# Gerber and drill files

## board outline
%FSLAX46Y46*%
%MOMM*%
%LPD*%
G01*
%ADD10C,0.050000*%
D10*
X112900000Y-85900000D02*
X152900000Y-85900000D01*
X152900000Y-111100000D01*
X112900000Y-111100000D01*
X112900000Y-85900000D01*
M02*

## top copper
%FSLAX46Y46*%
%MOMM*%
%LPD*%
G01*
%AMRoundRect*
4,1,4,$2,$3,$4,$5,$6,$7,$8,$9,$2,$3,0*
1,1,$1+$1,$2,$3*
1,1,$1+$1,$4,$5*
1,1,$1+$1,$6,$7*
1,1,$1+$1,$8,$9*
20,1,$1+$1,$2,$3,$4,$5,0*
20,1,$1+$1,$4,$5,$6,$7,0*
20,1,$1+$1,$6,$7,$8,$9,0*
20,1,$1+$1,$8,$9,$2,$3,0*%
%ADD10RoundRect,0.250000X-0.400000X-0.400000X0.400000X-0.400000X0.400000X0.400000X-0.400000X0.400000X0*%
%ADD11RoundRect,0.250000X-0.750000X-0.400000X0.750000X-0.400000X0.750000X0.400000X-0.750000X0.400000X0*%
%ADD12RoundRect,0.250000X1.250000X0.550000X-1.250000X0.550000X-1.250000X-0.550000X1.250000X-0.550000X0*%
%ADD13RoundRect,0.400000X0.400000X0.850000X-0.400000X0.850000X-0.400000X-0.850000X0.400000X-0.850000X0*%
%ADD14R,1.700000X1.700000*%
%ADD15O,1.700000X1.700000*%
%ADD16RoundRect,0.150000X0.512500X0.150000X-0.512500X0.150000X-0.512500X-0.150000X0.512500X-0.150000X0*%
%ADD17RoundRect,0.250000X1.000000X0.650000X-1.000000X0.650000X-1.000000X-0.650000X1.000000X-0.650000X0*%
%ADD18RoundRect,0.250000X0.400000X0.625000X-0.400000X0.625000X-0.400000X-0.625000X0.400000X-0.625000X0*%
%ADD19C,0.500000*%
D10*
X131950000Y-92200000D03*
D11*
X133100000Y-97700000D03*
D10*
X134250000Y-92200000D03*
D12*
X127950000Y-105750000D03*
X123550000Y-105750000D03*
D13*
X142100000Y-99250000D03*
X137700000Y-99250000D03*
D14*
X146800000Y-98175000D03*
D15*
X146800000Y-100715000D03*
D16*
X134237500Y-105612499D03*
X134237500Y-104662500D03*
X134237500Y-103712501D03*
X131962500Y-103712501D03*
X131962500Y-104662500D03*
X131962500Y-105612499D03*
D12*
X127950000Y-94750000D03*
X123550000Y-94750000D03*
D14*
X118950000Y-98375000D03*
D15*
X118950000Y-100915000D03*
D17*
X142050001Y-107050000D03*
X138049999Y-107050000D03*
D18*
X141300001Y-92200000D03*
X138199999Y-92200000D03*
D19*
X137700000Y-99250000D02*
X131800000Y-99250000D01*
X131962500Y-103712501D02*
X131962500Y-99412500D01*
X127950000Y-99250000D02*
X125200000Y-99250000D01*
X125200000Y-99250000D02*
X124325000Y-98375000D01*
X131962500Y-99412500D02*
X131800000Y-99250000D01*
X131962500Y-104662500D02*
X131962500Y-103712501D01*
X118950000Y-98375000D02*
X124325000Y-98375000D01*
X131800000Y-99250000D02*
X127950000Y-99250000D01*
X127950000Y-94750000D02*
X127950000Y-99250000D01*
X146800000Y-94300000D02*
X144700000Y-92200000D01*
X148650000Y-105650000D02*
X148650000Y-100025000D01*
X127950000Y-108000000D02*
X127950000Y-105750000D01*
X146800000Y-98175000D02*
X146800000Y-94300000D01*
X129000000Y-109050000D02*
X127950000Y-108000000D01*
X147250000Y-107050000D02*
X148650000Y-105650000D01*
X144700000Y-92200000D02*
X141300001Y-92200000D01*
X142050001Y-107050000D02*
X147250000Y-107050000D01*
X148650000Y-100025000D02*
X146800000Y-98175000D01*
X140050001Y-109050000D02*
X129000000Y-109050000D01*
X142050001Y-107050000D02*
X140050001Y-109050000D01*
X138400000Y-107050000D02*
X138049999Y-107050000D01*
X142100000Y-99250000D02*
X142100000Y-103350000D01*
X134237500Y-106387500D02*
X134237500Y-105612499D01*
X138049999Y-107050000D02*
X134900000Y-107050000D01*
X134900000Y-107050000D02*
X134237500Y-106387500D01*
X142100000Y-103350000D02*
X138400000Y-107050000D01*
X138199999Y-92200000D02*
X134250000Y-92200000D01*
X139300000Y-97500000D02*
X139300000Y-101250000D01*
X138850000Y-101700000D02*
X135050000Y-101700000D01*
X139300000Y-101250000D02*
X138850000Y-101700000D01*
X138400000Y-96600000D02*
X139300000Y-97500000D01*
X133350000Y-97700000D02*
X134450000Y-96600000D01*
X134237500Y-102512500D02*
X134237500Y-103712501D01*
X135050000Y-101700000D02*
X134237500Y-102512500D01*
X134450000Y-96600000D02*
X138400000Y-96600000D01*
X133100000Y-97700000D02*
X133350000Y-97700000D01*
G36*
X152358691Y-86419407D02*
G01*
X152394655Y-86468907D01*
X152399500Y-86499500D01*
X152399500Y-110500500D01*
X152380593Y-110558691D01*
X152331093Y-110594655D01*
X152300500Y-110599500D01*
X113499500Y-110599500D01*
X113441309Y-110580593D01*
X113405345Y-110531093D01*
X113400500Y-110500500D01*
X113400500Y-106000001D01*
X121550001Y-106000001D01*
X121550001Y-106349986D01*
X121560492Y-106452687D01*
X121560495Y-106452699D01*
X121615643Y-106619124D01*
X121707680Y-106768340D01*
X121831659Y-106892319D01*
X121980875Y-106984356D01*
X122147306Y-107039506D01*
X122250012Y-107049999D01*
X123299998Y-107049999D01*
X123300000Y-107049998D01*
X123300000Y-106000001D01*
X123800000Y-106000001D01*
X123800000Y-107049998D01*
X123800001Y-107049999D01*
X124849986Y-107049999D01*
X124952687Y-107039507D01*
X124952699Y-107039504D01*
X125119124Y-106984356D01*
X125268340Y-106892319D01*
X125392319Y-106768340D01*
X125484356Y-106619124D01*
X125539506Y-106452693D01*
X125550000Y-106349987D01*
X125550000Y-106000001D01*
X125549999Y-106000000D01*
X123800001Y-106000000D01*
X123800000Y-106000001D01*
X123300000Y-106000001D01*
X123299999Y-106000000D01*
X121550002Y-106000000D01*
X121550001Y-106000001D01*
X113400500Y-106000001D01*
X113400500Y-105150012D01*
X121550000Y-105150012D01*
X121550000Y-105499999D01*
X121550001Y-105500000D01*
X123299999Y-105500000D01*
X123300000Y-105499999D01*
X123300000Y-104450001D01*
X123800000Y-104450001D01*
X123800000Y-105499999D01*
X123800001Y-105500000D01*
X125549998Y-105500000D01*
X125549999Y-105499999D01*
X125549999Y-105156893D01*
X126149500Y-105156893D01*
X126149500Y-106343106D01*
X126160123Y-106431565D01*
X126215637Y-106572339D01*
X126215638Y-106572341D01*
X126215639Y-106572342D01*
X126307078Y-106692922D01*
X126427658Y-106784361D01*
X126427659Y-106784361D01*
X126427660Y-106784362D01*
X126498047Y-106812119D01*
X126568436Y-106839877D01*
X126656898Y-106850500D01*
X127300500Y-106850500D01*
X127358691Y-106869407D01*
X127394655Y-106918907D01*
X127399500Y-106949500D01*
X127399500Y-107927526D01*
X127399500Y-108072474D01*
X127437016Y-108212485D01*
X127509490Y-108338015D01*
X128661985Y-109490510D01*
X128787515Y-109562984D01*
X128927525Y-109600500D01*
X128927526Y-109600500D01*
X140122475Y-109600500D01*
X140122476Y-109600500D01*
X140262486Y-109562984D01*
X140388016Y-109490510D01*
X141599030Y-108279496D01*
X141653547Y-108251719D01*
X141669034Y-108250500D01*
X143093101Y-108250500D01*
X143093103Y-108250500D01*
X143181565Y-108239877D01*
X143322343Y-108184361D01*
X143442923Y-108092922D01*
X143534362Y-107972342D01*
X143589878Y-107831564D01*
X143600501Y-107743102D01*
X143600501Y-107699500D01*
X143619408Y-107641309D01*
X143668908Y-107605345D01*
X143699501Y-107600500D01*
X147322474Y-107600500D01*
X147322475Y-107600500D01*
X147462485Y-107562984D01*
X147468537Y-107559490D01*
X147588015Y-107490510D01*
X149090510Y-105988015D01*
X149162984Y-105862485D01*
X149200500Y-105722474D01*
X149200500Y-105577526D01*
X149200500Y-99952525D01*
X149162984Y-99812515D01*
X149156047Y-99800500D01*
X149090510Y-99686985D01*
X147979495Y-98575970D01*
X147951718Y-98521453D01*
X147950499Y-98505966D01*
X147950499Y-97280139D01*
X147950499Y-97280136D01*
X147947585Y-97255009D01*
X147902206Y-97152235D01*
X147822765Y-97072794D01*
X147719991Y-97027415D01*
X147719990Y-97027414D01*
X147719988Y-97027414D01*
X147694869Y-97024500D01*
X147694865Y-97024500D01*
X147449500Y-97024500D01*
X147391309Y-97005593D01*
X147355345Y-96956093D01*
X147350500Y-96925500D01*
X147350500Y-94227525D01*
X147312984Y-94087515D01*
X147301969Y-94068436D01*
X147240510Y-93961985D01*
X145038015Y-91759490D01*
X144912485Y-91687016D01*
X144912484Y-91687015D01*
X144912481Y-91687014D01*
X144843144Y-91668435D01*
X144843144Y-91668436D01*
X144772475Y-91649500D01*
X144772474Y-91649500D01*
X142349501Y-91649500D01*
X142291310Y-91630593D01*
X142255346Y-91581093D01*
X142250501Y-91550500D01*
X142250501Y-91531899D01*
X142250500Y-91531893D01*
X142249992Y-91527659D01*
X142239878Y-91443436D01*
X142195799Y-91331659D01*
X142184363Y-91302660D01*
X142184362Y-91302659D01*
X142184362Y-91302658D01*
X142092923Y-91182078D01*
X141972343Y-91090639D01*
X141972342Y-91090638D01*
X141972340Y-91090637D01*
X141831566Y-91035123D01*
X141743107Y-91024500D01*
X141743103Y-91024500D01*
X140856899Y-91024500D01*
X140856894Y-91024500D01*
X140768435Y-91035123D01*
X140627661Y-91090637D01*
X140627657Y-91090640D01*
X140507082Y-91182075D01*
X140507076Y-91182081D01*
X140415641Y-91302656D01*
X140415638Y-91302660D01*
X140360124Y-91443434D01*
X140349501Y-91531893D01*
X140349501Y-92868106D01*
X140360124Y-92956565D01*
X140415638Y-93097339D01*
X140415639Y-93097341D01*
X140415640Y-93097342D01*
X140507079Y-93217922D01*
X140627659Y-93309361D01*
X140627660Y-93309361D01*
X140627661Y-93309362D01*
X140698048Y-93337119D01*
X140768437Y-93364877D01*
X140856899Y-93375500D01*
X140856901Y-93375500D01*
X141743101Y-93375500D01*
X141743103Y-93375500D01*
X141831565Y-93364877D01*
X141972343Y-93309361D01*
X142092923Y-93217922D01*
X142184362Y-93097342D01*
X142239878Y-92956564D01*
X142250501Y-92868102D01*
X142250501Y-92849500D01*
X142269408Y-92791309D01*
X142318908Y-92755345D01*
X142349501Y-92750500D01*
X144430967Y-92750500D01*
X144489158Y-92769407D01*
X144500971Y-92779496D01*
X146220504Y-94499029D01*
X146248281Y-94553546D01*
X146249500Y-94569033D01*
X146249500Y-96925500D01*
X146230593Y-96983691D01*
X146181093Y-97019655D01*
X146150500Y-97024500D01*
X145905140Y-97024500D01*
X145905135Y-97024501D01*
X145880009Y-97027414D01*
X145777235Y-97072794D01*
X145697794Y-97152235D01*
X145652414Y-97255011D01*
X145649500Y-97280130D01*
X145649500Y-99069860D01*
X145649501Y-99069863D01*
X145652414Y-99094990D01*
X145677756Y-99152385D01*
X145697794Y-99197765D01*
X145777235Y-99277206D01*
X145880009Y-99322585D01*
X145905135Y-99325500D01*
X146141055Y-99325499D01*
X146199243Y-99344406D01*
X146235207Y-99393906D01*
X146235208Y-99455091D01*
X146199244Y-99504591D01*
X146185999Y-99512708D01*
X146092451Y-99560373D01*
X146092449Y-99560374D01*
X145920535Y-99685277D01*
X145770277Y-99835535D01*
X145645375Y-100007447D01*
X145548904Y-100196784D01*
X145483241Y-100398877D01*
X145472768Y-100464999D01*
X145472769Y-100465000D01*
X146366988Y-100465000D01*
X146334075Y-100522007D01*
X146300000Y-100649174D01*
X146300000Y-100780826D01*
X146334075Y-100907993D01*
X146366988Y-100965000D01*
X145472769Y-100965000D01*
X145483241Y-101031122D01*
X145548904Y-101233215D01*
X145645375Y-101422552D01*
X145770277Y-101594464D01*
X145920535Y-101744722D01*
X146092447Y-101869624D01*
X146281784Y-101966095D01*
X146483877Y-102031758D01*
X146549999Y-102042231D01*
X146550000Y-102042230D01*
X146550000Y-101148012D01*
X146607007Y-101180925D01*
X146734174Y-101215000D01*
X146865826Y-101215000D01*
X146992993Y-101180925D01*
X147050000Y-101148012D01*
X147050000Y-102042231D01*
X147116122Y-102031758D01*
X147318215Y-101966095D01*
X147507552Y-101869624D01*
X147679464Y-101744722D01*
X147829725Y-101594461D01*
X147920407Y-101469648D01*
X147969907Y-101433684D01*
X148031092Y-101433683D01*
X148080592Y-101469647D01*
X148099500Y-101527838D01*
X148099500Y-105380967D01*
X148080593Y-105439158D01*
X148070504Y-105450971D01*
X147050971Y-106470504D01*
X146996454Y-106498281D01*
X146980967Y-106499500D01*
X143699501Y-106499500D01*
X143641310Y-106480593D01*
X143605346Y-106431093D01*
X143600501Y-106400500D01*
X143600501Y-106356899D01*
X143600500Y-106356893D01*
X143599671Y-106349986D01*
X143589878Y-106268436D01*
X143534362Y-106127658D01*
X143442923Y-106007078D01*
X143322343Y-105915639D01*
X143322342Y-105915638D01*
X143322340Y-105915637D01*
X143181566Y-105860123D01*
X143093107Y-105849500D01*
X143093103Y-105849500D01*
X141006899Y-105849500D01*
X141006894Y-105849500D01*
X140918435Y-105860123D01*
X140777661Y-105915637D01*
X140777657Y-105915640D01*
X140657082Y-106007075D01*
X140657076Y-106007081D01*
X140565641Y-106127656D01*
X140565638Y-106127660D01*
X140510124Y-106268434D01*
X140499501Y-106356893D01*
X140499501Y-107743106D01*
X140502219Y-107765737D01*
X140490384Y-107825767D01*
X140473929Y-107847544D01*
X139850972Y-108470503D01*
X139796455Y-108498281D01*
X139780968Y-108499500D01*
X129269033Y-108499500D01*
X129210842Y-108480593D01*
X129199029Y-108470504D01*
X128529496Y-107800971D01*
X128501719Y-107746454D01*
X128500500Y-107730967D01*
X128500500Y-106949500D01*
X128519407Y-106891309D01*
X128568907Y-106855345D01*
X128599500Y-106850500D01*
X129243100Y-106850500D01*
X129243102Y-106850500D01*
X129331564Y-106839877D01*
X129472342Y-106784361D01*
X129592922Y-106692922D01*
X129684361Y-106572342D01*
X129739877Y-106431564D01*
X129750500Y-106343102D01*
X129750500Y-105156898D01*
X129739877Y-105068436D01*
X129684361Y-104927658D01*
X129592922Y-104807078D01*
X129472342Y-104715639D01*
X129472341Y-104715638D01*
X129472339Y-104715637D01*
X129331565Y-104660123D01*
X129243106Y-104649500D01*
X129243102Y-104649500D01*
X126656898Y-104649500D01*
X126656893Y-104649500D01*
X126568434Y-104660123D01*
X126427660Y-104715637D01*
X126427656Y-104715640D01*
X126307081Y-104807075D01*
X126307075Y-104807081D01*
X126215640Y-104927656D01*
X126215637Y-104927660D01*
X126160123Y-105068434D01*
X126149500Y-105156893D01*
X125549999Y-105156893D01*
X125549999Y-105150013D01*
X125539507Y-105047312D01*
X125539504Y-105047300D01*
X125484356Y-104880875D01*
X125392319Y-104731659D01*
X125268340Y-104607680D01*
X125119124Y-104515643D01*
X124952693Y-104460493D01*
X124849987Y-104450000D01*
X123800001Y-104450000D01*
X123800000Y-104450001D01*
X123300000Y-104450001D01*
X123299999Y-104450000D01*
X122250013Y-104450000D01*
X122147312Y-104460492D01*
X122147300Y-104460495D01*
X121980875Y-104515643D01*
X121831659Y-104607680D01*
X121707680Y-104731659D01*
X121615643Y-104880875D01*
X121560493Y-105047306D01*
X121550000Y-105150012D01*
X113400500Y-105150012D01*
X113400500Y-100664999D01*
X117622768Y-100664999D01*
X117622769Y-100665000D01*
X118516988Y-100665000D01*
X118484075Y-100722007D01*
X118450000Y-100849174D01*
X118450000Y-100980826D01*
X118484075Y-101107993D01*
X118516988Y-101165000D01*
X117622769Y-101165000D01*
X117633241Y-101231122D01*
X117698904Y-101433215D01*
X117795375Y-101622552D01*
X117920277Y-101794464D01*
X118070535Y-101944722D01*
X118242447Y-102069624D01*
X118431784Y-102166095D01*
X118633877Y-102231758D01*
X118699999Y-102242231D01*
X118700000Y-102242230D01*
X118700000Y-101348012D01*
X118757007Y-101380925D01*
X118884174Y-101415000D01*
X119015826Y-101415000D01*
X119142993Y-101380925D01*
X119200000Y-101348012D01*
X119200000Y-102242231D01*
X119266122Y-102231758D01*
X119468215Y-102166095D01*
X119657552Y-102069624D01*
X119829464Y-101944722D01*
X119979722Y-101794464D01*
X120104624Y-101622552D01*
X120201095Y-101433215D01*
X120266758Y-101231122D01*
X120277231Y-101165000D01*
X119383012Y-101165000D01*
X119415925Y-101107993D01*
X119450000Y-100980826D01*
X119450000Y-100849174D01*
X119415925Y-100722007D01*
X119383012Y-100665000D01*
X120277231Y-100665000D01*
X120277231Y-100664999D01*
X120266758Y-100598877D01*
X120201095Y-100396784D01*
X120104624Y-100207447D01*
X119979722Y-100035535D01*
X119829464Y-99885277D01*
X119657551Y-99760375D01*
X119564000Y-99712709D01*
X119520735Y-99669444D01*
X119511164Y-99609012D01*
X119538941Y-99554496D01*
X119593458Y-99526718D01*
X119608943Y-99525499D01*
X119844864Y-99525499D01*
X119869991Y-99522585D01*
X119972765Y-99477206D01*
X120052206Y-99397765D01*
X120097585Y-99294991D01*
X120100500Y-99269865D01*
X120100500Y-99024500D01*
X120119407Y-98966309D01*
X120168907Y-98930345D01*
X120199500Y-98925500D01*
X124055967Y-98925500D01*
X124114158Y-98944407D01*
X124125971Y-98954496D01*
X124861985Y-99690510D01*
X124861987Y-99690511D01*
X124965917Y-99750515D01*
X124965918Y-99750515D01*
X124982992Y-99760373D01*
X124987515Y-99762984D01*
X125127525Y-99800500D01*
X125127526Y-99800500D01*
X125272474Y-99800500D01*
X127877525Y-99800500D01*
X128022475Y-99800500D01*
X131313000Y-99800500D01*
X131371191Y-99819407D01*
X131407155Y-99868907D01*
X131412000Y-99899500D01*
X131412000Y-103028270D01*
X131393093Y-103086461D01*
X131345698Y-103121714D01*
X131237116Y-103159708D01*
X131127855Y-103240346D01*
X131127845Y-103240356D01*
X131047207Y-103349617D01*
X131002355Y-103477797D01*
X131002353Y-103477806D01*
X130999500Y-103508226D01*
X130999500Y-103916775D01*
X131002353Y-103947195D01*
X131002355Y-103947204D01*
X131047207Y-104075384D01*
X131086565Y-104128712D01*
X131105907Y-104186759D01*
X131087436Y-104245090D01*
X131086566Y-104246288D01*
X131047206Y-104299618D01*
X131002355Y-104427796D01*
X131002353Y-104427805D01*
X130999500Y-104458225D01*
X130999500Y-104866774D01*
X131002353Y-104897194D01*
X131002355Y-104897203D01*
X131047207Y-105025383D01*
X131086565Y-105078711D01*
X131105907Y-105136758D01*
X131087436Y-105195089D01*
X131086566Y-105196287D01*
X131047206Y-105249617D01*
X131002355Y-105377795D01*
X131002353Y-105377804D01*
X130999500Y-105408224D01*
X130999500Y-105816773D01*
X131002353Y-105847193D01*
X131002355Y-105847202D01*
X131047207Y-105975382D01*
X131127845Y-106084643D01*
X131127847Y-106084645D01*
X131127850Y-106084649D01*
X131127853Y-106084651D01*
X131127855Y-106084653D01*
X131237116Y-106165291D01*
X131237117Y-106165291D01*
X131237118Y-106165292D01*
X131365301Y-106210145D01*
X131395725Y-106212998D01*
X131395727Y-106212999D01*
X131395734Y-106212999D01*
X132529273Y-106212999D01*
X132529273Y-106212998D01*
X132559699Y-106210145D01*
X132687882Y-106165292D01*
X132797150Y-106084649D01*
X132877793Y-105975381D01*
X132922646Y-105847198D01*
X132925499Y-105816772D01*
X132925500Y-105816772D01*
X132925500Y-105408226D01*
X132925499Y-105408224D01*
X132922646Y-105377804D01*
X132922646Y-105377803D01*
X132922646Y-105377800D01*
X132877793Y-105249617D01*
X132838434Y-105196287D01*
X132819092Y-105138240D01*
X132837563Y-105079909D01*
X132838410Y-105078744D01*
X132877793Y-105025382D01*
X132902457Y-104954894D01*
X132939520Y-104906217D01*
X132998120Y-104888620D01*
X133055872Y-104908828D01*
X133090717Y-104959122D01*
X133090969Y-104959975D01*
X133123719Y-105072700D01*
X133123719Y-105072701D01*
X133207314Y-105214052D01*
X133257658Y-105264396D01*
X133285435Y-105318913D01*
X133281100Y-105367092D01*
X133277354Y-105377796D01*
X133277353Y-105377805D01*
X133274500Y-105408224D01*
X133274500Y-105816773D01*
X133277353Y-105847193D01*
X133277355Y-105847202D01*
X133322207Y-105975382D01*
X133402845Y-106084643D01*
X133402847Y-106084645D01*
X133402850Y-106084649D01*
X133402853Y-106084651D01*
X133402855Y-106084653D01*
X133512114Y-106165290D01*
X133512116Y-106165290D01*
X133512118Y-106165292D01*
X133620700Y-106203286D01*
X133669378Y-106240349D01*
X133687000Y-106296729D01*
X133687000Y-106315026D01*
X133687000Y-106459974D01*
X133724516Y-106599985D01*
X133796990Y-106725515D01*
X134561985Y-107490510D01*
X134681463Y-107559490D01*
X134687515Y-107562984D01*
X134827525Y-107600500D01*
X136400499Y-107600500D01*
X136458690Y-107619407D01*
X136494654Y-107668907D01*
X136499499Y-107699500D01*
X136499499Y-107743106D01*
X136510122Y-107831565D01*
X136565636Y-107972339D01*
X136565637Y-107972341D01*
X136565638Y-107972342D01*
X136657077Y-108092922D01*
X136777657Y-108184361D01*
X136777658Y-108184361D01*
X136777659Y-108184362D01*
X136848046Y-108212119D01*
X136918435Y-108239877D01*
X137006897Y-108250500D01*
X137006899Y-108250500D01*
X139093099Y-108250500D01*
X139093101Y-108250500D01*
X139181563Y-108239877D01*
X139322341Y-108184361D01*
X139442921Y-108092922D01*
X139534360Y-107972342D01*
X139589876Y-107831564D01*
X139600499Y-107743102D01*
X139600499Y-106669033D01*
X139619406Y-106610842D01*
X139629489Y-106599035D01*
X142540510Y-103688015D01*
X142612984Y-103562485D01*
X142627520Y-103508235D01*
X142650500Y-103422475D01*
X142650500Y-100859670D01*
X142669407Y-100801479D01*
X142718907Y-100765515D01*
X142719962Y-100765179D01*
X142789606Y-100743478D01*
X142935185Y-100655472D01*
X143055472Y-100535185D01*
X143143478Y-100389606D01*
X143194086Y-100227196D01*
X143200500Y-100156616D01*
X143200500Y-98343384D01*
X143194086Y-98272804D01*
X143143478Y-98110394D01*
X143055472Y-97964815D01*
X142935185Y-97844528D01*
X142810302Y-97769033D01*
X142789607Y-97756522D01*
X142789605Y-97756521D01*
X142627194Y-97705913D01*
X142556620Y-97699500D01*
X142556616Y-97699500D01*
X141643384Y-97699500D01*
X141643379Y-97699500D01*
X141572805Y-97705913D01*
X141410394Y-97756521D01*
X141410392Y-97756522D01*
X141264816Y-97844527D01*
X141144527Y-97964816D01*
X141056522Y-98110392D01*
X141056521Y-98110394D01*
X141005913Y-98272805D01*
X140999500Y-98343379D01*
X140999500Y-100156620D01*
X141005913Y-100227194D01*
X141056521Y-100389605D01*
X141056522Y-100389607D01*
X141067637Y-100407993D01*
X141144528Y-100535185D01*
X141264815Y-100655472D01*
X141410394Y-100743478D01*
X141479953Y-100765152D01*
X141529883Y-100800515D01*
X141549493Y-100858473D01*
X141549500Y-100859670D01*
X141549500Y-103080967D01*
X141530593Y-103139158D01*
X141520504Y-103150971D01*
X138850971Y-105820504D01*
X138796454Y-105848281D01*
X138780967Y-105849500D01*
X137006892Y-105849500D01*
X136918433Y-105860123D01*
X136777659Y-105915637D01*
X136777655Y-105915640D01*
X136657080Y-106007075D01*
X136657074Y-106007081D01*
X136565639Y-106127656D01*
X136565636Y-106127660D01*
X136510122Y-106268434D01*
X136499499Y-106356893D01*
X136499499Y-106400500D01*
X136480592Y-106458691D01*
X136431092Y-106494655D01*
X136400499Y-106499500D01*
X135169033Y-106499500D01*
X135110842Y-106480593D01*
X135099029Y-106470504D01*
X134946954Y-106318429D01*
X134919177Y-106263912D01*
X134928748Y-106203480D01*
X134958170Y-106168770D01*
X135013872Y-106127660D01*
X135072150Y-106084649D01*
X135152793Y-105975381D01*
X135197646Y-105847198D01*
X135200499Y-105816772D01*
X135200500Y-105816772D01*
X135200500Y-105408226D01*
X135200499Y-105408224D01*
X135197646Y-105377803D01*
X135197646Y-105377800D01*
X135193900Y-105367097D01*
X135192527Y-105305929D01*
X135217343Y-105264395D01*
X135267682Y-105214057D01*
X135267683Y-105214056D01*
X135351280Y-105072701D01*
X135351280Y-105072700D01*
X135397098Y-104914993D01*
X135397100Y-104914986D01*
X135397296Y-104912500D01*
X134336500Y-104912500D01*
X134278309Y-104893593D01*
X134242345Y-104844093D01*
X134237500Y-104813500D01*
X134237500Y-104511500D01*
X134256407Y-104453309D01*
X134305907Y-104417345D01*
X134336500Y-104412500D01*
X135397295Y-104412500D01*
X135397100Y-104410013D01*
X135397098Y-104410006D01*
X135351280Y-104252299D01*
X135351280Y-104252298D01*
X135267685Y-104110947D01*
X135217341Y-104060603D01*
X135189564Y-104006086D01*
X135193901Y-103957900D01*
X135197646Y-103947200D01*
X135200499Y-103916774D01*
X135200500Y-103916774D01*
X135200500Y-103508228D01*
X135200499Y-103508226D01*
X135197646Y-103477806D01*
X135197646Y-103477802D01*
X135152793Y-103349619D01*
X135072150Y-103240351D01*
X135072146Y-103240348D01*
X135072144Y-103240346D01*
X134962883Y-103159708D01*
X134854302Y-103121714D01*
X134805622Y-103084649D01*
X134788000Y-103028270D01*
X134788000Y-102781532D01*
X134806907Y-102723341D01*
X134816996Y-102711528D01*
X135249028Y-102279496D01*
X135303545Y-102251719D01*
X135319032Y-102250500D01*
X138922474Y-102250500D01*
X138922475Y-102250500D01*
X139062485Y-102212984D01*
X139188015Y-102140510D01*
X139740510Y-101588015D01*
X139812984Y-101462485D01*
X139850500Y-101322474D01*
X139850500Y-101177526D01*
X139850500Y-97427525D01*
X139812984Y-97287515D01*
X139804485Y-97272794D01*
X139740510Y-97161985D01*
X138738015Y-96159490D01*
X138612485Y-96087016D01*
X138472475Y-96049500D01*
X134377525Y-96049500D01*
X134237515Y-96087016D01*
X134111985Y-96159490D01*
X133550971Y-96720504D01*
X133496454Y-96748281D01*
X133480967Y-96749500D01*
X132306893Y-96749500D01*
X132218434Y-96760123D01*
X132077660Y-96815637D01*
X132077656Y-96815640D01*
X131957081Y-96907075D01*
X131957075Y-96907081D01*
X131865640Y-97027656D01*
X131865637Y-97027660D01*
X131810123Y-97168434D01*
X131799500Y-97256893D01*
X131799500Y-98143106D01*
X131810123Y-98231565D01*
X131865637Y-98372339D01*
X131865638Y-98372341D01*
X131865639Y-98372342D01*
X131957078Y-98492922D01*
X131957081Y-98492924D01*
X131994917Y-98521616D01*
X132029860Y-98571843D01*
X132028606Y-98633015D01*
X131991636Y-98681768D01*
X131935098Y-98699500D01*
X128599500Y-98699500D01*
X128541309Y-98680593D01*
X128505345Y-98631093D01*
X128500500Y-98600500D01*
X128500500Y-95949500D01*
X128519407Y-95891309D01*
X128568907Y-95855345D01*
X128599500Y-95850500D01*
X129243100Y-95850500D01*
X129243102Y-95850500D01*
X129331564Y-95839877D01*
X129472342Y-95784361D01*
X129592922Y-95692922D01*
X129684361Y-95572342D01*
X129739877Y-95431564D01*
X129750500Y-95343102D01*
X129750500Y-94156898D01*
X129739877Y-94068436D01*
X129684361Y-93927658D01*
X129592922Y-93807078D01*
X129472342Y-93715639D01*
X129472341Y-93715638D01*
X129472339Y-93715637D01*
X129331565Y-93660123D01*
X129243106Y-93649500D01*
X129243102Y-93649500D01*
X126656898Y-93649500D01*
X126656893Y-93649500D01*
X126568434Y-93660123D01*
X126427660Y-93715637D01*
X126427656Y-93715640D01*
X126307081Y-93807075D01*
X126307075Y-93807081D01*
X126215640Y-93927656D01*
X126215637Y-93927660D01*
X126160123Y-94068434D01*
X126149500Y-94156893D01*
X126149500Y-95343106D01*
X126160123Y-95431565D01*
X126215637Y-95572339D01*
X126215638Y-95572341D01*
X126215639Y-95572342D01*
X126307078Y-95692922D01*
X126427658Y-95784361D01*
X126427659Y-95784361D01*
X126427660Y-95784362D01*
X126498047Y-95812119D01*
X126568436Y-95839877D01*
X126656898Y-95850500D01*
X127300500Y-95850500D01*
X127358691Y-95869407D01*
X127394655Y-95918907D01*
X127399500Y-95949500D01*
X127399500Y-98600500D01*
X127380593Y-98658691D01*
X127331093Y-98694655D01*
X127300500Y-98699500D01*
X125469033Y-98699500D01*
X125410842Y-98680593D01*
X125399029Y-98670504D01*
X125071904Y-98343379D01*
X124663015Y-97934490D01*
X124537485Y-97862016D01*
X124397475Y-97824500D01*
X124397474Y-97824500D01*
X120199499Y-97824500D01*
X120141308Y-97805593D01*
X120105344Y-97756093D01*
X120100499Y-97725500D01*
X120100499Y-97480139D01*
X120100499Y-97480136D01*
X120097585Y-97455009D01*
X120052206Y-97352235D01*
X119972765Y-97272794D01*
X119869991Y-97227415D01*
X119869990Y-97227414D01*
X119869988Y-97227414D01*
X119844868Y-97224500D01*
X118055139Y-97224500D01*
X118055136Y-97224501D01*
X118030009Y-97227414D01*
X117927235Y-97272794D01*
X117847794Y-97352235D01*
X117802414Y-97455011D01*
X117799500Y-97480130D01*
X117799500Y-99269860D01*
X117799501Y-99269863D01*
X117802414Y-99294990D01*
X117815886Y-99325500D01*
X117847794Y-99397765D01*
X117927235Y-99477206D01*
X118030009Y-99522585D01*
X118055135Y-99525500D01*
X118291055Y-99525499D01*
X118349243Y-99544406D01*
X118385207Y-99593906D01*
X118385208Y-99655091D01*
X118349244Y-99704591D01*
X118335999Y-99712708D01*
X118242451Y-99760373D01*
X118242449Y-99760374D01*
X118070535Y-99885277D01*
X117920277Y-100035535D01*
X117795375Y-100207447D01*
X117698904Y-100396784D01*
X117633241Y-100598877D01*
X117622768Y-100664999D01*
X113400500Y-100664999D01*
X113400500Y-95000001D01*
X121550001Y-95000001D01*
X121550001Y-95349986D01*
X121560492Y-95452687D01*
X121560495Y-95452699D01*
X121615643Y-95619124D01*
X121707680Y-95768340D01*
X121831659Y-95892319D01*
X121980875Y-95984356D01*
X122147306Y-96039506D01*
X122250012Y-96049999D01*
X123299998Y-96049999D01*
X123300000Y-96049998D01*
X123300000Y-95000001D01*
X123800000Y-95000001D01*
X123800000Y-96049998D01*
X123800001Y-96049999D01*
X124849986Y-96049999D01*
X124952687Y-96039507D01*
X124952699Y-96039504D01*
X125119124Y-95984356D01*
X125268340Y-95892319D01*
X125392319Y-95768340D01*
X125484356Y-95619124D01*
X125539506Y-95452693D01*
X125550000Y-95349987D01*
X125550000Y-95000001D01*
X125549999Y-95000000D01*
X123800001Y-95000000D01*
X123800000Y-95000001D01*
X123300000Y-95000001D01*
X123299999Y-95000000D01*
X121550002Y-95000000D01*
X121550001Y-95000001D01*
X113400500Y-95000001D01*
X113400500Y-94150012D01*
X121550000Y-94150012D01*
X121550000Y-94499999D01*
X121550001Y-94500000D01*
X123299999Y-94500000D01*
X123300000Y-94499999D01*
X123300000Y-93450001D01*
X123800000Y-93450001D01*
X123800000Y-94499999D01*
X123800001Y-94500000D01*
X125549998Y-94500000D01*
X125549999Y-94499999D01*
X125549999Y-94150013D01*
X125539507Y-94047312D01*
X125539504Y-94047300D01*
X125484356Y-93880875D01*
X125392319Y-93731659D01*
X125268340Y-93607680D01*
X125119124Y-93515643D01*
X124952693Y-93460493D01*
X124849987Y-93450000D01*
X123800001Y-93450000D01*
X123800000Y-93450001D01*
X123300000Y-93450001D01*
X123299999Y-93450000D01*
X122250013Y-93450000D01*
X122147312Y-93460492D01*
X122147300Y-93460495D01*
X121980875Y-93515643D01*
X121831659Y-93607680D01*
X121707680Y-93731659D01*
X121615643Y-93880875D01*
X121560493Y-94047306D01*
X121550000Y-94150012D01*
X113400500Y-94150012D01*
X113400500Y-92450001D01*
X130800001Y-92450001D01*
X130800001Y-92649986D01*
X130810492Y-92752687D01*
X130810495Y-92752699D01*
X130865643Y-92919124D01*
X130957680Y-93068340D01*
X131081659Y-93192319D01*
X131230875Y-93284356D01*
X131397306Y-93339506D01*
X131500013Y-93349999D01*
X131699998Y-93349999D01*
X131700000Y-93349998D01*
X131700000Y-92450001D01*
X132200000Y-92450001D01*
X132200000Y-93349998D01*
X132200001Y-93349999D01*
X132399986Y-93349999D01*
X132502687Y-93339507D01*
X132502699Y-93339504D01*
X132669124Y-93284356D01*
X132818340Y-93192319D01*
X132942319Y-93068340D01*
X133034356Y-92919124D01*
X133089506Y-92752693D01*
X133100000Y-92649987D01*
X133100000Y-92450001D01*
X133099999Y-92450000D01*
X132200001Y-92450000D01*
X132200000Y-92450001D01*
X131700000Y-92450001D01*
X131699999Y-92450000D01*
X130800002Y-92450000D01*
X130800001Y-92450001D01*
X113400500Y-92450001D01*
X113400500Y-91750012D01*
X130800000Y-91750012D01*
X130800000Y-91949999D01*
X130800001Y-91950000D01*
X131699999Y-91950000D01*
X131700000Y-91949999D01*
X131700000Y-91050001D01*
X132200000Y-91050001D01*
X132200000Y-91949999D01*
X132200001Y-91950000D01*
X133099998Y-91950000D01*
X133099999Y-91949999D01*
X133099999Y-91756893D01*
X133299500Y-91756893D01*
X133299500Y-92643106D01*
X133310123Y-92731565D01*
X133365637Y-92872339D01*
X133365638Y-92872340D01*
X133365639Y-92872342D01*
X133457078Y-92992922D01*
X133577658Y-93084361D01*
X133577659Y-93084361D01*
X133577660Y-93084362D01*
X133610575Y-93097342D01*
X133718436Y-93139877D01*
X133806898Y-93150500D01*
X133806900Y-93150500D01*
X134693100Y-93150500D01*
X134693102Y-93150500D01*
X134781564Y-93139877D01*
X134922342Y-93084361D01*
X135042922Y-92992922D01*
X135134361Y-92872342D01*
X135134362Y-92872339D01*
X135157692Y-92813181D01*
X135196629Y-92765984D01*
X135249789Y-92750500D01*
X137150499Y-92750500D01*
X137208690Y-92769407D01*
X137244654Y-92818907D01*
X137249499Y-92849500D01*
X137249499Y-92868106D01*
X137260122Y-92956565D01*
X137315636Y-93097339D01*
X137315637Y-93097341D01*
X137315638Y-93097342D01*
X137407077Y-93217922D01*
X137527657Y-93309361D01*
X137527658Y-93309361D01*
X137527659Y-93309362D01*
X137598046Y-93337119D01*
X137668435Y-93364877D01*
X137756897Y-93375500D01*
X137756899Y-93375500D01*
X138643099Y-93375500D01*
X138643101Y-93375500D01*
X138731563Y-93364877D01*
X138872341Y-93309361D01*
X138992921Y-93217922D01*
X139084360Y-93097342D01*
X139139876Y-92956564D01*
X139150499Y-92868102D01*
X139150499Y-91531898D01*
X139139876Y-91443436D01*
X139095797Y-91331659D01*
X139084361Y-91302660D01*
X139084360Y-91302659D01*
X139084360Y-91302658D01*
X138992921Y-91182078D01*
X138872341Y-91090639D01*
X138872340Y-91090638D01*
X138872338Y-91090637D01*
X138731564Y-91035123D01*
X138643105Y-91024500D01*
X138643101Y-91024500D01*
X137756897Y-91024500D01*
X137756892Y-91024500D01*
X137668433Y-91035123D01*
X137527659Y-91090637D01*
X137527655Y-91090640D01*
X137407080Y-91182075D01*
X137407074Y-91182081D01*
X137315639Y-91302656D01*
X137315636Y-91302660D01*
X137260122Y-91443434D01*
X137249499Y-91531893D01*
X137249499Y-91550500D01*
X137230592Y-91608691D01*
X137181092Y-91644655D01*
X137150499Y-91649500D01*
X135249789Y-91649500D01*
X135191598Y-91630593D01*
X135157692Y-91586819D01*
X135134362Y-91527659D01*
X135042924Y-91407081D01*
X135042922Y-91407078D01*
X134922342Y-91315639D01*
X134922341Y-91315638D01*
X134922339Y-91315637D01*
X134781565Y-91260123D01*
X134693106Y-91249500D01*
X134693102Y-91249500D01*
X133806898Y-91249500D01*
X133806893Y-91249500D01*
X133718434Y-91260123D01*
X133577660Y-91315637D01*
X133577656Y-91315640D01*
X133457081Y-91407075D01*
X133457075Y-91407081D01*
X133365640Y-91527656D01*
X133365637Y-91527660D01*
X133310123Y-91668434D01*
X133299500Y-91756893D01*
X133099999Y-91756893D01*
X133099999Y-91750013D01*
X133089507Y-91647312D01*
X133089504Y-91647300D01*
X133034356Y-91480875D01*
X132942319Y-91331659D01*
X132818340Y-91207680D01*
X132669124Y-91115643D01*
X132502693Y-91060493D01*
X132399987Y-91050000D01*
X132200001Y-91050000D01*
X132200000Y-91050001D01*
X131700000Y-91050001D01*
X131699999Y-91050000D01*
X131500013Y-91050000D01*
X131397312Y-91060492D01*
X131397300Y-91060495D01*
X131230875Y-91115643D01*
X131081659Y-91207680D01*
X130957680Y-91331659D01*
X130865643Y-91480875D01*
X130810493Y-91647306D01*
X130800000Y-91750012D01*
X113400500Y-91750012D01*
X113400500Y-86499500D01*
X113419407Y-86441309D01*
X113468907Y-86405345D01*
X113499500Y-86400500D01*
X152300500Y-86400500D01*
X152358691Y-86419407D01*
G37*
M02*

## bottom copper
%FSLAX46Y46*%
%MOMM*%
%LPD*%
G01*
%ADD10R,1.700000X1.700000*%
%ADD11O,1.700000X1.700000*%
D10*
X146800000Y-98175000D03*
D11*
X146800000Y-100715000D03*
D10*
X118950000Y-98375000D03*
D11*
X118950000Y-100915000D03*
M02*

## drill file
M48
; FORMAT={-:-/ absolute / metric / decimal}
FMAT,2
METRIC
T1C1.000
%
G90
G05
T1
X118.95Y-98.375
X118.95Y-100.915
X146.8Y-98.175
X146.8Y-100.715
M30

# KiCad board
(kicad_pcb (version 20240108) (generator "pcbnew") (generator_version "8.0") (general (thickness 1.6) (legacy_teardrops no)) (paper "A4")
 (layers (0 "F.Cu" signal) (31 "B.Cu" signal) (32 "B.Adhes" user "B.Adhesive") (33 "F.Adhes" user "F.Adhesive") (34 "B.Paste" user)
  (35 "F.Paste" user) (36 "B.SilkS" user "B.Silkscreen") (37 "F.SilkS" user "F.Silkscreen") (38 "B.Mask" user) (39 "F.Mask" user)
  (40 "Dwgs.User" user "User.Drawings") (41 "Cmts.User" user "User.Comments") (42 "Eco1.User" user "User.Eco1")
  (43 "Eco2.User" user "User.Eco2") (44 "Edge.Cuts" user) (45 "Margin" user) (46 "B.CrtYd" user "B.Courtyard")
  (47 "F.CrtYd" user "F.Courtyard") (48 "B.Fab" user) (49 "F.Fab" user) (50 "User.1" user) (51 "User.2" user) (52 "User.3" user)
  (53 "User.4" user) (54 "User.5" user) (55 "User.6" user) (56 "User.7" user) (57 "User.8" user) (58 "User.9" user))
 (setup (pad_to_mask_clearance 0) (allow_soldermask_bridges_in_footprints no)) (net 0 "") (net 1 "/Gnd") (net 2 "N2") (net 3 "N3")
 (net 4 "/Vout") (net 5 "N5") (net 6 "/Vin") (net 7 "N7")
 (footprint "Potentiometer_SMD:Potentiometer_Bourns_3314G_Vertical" (layer "F.Cu") (at 133.1 94.95)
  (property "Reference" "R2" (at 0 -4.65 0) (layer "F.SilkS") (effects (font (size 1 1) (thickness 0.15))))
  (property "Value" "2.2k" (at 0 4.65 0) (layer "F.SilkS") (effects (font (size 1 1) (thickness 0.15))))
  (pad "1" smd roundrect (at -1.15 -2.75) (size 1.3 1.3) (layers "F.Cu" "F.Paste" "F.Mask") (roundrect_rratio 0.1923076923) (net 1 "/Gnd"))
  (pad "2" smd roundrect (at 0 2.75) (size 2 1.3) (layers "F.Cu" "F.Paste" "F.Mask") (roundrect_rratio 0.1923076923) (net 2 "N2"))
  (pad "3" smd roundrect (at 1.15 -2.75) (size 1.3 1.3) (layers "F.Cu" "F.Paste" "F.Mask") (roundrect_rratio 0.1923076923) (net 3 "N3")))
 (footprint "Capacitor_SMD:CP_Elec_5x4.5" (layer "F.Cu") (at 125.75 105.75 180)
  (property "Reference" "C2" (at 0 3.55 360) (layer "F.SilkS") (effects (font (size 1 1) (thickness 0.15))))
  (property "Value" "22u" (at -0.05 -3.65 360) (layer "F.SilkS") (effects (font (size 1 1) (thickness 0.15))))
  (pad "1" smd roundrect (at -2.2 0 180) (size 3 1.6) (layers "F.Cu" "F.Paste" "F.Mask") (roundrect_rratio 0.15625) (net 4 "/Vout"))
  (pad "2" smd roundrect (at 2.2 0 180) (size 3 1.6) (layers "F.Cu" "F.Paste" "F.Mask") (roundrect_rratio 0.15625) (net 1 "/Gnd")))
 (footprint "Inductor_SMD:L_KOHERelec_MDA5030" (layer "F.Cu") (at 139.9 99.25 180)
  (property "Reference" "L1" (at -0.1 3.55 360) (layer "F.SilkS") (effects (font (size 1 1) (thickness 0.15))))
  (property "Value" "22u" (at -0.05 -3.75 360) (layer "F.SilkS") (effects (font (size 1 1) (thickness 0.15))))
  (pad "1" smd roundrect (at -2.2 0 180) (size 1.6 2.5) (layers "F.Cu" "F.Paste" "F.Mask") (roundrect_rratio 0.25) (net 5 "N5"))
  (pad "2" smd roundrect (at 2.2 0 180) (size 1.6 2.5) (layers "F.Cu" "F.Paste" "F.Mask") (roundrect_rratio 0.25) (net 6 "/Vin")))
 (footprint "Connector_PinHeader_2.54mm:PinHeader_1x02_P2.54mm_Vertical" (layer "F.Cu") (at 146.8 98.175)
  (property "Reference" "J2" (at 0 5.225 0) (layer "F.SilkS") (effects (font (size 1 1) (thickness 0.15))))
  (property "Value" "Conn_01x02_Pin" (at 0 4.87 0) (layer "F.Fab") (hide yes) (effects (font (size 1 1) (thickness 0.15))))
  (pad "1" thru_hole rect (at 0 0) (size 1.7 1.7) (drill 1) (layers "*.Cu" "*.Mask") (remove_unused_layers no) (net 4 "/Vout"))
  (pad "2" thru_hole oval (at 0 2.54) (size 1.7 1.7) (drill 1) (layers "*.Cu" "*.Mask") (remove_unused_layers no) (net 1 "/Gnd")))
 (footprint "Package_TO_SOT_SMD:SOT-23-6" (layer "F.Cu") (at 133.1 104.6625 180)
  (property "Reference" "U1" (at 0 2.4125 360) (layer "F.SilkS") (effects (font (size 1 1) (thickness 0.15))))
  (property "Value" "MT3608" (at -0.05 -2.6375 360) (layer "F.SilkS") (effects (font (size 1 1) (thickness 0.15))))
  (pad "1" smd roundrect (at -1.1375 -0.949999 180) (size 1.325 0.6) (layers "F.Cu" "F.Paste" "F.Mask") (roundrect_rratio 0.25) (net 5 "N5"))
  (pad "2" smd roundrect (at -1.1375 0 180) (size 1.325 0.6) (layers "F.Cu" "F.Paste" "F.Mask") (roundrect_rratio 0.25) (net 1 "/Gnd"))
  (pad "3" smd roundrect (at -1.1375 0.949999 180) (size 1.325 0.6) (layers "F.Cu" "F.Paste" "F.Mask") (roundrect_rratio 0.25) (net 2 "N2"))
  (pad "4" smd roundrect (at 1.1375 0.949999 180) (size 1.325 0.6) (layers "F.Cu" "F.Paste" "F.Mask") (roundrect_rratio 0.25) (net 6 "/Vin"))
  (pad "5" smd roundrect (at 1.1375 0 180) (size 1.325 0.6) (layers "F.Cu" "F.Paste" "F.Mask") (roundrect_rratio 0.25) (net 6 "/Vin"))
  (pad "6" smd roundrect (at 1.1375 -0.949999 180) (size 1.325 0.6) (layers "F.Cu" "F.Paste" "F.Mask") (roundrect_rratio 0.25) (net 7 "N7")))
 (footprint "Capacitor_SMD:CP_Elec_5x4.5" (layer "F.Cu") (at 125.75 94.75 180)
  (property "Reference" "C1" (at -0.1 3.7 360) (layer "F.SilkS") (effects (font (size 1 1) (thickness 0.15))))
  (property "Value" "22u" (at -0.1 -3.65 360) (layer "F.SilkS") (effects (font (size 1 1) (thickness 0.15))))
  (pad "1" smd roundrect (at -2.2 0 180) (size 3 1.6) (layers "F.Cu" "F.Paste" "F.Mask") (roundrect_rratio 0.15625) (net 6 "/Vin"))
  (pad "2" smd roundrect (at 2.2 0 180) (size 3 1.6) (layers "F.Cu" "F.Paste" "F.Mask") (roundrect_rratio 0.15625) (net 1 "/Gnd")))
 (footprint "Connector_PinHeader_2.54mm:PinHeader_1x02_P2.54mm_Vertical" (layer "F.Cu") (at 118.95 98.375)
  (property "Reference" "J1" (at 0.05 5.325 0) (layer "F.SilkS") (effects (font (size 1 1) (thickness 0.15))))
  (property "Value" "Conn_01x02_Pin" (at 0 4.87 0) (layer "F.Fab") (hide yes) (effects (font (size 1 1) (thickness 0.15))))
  (pad "1" thru_hole rect (at 0 0) (size 1.7 1.7) (drill 1) (layers "*.Cu" "*.Mask") (remove_unused_layers no) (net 6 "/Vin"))
  (pad "2" thru_hole oval (at 0 2.54) (size 1.7 1.7) (drill 1) (layers "*.Cu" "*.Mask") (remove_unused_layers no) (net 1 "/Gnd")))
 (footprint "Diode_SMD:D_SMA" (layer "F.Cu") (at 140.05 107.05 180)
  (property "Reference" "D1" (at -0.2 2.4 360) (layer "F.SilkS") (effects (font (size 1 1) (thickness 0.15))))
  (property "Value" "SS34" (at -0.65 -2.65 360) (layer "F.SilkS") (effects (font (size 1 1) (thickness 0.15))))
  (pad "1" smd roundrect (at -2.000001 0 180) (size 2.5 1.8) (layers "F.Cu" "F.Paste" "F.Mask") (roundrect_rratio 0.1388888889)
   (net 4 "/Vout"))
  (pad "2" smd roundrect (at 2.000001 0 180) (size 2.5 1.8) (layers "F.Cu" "F.Paste" "F.Mask") (roundrect_rratio 0.1388888889) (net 5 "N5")))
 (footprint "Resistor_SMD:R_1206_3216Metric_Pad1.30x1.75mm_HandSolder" (layer "F.Cu") (at 139.75 92.2 180)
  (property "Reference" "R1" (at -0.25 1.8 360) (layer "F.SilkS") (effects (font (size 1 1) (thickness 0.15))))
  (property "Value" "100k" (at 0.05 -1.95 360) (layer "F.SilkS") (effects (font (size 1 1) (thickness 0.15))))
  (pad "1" smd roundrect (at -1.550001 0 180) (size 1.3 1.75) (layers "F.Cu" "F.Paste" "F.Mask") (roundrect_rratio 0.192308) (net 4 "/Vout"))
  (pad "2" smd roundrect (at 1.550001 0 180) (size 1.3 1.75) (layers "F.Cu" "F.Paste" "F.Mask") (roundrect_rratio 0.192308) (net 3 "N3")))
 (gr_rect (start 112.9 85.9) (end 152.9 111.1) (stroke (width 0.05) (type default)) (fill none) (layer "Edge.Cuts"))
 (segment (start 137.7 99.25) (end 131.8 99.25) (width 0.5) (layer "F.Cu") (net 6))
 (segment (start 131.9625 103.712501) (end 131.9625 99.4125) (width 0.5) (layer "F.Cu") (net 6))
 (segment (start 127.95 99.25) (end 125.2 99.25) (width 0.5) (layer "F.Cu") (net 6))
 (segment (start 125.2 99.25) (end 124.325 98.375) (width 0.5) (layer "F.Cu") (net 6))
 (segment (start 131.9625 99.4125) (end 131.8 99.25) (width 0.5) (layer "F.Cu") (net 6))
 (segment (start 131.9625 104.6625) (end 131.9625 103.712501) (width 0.5) (layer "F.Cu") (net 6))
 (segment (start 118.95 98.375) (end 124.325 98.375) (width 0.5) (layer "F.Cu") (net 6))
 (segment (start 131.8 99.25) (end 127.95 99.25) (width 0.5) (layer "F.Cu") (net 6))
 (segment (start 127.95 94.75) (end 127.95 99.25) (width 0.5) (layer "F.Cu") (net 6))
 (segment (start 146.8 94.3) (end 144.7 92.2) (width 0.5) (layer "F.Cu") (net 4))
 (segment (start 148.65 105.65) (end 148.65 100.025) (width 0.5) (layer "F.Cu") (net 4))
 (segment (start 127.95 108) (end 127.95 105.75) (width 0.5) (layer "F.Cu") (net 4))
 (segment (start 146.8 98.175) (end 146.8 94.3) (width 0.5) (layer "F.Cu") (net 4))
 (segment (start 129 109.05) (end 127.95 108) (width 0.5) (layer "F.Cu") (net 4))
 (segment (start 147.25 107.05) (end 148.65 105.65) (width 0.5) (layer "F.Cu") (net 4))
 (segment (start 144.7 92.2) (end 141.300001 92.2) (width 0.5) (layer "F.Cu") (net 4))
 (segment (start 142.050001 107.05) (end 147.25 107.05) (width 0.5) (layer "F.Cu") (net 4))
 (segment (start 148.65 100.025) (end 146.8 98.175) (width 0.5) (layer "F.Cu") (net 4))
 (segment (start 140.050001 109.05) (end 129 109.05) (width 0.5) (layer "F.Cu") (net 4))
 (segment (start 142.050001 107.05) (end 140.050001 109.05) (width 0.5) (layer "F.Cu") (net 4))
 (segment (start 138.4 107.05) (end 138.049999 107.05) (width 0.5) (layer "F.Cu") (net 5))
 (segment (start 142.1 99.25) (end 142.1 103.35) (width 0.5) (layer "F.Cu") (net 5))
 (segment (start 134.2375 106.3875) (end 134.2375 105.612499) (width 0.5) (layer "F.Cu") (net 5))
 (segment (start 138.049999 107.05) (end 134.9 107.05) (width 0.5) (layer "F.Cu") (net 5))
 (segment (start 134.9 107.05) (end 134.2375 106.3875) (width 0.5) (layer "F.Cu") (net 5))
 (segment (start 142.1 103.35) (end 138.4 107.05) (width 0.5) (layer "F.Cu") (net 5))
 (segment (start 138.199999 92.2) (end 134.25 92.2) (width 0.5) (layer "F.Cu") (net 3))
 (segment (start 139.3 97.5) (end 139.3 101.25) (width 0.5) (layer "F.Cu") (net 2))
 (segment (start 138.85 101.7) (end 135.05 101.7) (width 0.5) (layer "F.Cu") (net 2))
 (segment (start 139.3 101.25) (end 138.85 101.7) (width 0.5) (layer "F.Cu") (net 2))
 (segment (start 138.4 96.6) (end 139.3 97.5) (width 0.5) (layer "F.Cu") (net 2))
 (segment (start 133.35 97.7) (end 134.45 96.6) (width 0.5) (layer "F.Cu") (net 2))
 (segment (start 134.2375 102.5125) (end 134.2375 103.712501) (width 0.5) (layer "F.Cu") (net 2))
 (segment (start 135.05 101.7) (end 134.2375 102.5125) (width 0.5) (layer "F.Cu") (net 2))
 (segment (start 134.45 96.6) (end 138.4 96.6) (width 0.5) (layer "F.Cu") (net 2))
 (segment (start 133.1 97.7) (end 133.35 97.7) (width 0.5) (layer "F.Cu") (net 2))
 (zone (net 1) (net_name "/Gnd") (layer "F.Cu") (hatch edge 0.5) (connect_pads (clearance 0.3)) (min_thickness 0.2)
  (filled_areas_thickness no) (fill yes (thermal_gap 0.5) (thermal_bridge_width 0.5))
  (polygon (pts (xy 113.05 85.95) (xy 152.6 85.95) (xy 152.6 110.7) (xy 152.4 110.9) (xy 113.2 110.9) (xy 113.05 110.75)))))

